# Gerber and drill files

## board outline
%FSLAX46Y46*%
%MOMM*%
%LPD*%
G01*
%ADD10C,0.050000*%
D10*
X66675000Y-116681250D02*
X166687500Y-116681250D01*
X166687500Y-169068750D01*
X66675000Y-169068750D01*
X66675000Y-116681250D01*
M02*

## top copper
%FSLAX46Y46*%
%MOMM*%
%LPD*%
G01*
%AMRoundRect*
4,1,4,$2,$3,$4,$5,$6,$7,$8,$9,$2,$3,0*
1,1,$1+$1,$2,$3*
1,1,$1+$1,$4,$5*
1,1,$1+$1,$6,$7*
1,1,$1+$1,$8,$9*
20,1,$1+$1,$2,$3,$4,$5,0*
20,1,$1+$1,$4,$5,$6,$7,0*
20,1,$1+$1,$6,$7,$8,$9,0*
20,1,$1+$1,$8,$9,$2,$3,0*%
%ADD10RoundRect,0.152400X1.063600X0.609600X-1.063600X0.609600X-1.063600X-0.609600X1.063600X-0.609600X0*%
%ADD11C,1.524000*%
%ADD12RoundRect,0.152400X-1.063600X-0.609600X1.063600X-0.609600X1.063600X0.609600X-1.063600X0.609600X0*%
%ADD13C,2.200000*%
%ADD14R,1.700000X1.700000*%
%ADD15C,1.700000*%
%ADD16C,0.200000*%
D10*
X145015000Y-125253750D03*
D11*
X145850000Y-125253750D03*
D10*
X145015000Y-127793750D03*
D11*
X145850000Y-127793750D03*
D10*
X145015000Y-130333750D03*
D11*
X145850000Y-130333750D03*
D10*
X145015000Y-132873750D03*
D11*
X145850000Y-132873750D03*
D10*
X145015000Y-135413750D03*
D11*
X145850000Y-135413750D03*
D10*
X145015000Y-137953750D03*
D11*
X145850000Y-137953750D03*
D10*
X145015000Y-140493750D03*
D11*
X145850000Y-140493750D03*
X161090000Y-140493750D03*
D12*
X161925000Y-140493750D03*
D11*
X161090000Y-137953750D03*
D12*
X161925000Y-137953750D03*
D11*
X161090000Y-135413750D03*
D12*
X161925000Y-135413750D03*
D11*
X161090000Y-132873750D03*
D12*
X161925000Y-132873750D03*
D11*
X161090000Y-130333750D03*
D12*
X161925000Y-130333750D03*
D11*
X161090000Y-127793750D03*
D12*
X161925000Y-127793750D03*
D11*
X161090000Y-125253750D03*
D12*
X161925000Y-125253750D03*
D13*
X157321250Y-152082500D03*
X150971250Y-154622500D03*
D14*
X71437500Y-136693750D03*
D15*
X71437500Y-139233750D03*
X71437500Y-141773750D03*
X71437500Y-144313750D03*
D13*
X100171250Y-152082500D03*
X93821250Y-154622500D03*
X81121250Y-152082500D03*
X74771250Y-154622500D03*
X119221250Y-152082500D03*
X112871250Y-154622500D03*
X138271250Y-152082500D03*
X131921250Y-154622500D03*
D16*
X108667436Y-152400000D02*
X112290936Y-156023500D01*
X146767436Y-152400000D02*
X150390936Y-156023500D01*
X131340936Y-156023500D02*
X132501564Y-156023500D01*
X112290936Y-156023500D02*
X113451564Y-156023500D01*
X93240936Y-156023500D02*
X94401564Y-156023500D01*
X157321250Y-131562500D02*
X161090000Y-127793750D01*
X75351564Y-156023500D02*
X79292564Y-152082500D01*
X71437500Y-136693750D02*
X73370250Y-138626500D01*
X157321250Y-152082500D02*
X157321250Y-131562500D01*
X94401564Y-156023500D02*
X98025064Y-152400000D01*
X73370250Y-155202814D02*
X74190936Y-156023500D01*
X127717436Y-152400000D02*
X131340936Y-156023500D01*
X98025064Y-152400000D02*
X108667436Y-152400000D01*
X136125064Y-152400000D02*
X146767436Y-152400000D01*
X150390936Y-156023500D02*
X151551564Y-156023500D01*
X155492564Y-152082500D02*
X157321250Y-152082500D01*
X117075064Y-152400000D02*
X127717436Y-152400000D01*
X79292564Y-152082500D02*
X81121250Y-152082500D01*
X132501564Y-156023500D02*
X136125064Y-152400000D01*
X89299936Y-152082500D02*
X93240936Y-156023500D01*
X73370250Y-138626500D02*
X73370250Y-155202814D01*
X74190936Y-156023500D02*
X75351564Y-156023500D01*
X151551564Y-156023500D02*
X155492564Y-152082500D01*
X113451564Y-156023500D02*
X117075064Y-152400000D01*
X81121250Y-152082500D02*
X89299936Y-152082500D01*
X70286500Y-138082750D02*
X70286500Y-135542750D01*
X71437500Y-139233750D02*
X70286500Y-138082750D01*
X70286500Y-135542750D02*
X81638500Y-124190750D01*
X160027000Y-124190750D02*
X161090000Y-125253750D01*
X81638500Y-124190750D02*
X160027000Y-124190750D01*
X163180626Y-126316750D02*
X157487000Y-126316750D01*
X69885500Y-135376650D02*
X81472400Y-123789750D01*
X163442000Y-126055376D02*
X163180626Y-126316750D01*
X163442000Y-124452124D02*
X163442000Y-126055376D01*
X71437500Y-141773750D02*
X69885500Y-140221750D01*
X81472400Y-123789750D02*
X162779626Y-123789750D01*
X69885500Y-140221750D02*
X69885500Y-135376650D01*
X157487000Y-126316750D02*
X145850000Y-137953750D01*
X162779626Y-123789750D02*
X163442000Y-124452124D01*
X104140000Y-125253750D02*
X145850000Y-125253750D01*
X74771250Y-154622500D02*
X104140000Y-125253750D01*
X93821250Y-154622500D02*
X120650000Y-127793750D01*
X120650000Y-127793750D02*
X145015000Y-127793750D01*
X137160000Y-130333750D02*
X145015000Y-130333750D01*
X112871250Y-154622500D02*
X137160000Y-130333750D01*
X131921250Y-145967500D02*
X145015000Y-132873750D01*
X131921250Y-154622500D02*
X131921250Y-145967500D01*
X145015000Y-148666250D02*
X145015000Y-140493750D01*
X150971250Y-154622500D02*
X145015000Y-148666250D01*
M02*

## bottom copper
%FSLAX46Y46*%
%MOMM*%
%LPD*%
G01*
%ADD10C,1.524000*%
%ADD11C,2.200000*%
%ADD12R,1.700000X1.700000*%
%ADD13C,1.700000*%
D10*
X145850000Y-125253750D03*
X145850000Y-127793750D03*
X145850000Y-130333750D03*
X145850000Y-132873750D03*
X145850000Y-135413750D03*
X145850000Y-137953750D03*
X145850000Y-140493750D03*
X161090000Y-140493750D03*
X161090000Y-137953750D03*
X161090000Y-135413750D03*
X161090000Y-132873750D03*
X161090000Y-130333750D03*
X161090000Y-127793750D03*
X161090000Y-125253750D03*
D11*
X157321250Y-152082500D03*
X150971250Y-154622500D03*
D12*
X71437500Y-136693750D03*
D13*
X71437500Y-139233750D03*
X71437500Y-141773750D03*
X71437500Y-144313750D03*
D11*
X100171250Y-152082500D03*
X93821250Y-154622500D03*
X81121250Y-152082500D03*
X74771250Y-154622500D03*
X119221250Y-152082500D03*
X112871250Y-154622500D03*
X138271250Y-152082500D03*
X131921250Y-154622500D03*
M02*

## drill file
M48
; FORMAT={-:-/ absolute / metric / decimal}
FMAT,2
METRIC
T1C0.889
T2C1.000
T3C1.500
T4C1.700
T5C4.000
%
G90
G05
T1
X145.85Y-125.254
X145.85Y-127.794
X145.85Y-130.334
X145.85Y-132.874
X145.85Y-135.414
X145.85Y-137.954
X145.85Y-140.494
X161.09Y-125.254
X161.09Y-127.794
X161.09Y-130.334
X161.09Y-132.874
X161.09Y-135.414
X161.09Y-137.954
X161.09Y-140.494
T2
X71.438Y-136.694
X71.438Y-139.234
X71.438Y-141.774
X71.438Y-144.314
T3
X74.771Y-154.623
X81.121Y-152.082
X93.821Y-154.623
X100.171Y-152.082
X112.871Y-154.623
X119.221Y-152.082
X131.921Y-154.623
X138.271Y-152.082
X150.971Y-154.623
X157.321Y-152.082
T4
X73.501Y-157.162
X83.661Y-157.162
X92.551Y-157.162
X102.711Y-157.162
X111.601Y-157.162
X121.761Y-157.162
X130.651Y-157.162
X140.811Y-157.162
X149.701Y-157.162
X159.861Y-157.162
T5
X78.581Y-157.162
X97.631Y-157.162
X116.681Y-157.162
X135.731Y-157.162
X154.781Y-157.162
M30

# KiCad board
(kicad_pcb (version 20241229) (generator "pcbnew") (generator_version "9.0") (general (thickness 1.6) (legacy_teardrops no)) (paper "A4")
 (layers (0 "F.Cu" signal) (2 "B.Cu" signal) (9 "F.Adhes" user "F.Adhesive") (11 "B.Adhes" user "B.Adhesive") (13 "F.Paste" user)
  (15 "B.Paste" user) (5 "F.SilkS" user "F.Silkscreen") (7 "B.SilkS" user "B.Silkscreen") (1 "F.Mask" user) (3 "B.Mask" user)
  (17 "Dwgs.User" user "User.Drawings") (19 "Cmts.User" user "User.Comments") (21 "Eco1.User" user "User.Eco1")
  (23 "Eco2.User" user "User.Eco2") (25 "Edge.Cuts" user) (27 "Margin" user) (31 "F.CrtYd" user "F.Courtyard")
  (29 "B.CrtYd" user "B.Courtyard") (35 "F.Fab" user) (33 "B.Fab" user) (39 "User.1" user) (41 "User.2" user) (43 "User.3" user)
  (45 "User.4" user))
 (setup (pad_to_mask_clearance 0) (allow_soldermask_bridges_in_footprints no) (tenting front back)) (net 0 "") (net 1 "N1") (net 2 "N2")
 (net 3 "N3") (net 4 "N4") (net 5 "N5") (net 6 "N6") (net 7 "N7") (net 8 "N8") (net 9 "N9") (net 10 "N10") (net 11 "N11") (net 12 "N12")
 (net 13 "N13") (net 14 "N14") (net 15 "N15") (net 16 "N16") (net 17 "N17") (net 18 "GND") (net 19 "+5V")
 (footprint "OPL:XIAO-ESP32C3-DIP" (layer "F.Cu") (at 153.59 132.87375)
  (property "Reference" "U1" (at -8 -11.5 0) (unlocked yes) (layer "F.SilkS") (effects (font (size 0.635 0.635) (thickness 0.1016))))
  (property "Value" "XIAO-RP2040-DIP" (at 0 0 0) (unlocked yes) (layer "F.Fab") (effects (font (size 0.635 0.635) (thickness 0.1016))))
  (pad "1" smd roundrect (at -8.575 -7.62 180) (size 2.432 1.524) (layers "F.Cu" "F.Mask") (roundrect_rratio 0.1) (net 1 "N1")
   (thermal_bridge_angle 45))
  (pad "1" thru_hole circle (at -7.74 -7.62 180) (size 1.524 1.524) (drill 0.889) (layers "*.Cu" "*.Mask") (remove_unused_layers no)
   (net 1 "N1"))
  (pad "2" smd roundrect (at -8.575 -5.08 180) (size 2.432 1.524) (layers "F.Cu" "F.Mask") (roundrect_rratio 0.1) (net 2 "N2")
   (thermal_bridge_angle 45))
  (pad "2" thru_hole circle (at -7.74 -5.08 180) (size 1.524 1.524) (drill 0.889) (layers "*.Cu" "*.Mask") (remove_unused_layers no)
   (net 2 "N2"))
  (pad "3" smd roundrect (at -8.575 -2.54 180) (size 2.432 1.524) (layers "F.Cu" "F.Mask") (roundrect_rratio 0.1) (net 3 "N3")
   (thermal_bridge_angle 45))
  (pad "3" thru_hole circle (at -7.74 -2.54 180) (size 1.524 1.524) (drill 0.889) (layers "*.Cu" "*.Mask") (remove_unused_layers no)
   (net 3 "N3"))
  (pad "4" smd roundrect (at -8.575 0 180) (size 2.432 1.524) (layers "F.Cu" "F.Mask") (roundrect_rratio 0.1) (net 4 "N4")
   (thermal_bridge_angle 45))
  (pad "4" thru_hole circle (at -7.74 0 180) (size 1.524 1.524) (drill 0.889) (layers "*.Cu" "*.Mask") (remove_unused_layers no)
   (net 4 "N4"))
  (pad "5" smd roundrect (at -8.575 2.54 180) (size 2.432 1.524) (layers "F.Cu" "F.Mask") (roundrect_rratio 0.1) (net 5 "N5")
   (thermal_bridge_angle 45))
  (pad "5" thru_hole circle (at -7.74 2.54 180) (size 1.524 1.524) (drill 0.889) (layers "*.Cu" "*.Mask") (remove_unused_layers no)
   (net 5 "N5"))
  (pad "6" smd roundrect (at -8.575 5.08 180) (size 2.432 1.524) (layers "F.Cu" "F.Mask") (roundrect_rratio 0.1) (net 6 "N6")
   (thermal_bridge_angle 45))
  (pad "6" thru_hole circle (at -7.74 5.08 180) (size 1.524 1.524) (drill 0.889) (layers "*.Cu" "*.Mask") (remove_unused_layers no)
   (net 6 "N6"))
  (pad "7" smd roundrect (at -8.575 7.62 180) (size 2.432 1.524) (layers "F.Cu" "F.Mask") (roundrect_rratio 0.1) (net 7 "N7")
   (thermal_bridge_angle 45))
  (pad "7" thru_hole circle (at -7.74 7.62 180) (size 1.524 1.524) (drill 0.889) (layers "*.Cu" "*.Mask") (remove_unused_layers no)
   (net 7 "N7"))
  (pad "8" thru_hole circle (at 7.5 7.62) (size 1.524 1.524) (drill 0.889) (layers "*.Cu" "*.Mask") (remove_unused_layers no) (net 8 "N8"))
  (pad "8" smd roundrect (at 8.335 7.62) (size 2.432 1.524) (layers "F.Cu" "F.Mask") (roundrect_rratio 0.1) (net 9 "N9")
   (thermal_bridge_angle 45))
  (pad "9" thru_hole circle (at 7.5 5.08) (size 1.524 1.524) (drill 0.889) (layers "*.Cu" "*.Mask") (remove_unused_layers no) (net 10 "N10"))
  (pad "9" smd roundrect (at 8.335 5.08) (size 2.432 1.524) (layers "F.Cu" "F.Mask") (roundrect_rratio 0.1) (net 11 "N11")
   (thermal_bridge_angle 45))
  (pad "10" thru_hole circle (at 7.5 2.54) (size 1.524 1.524) (drill 0.889) (layers "*.Cu" "*.Mask") (remove_unused_layers no)
   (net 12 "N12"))
  (pad "10" smd roundrect (at 8.335 2.54) (size 2.432 1.524) (layers "F.Cu" "F.Mask") (roundrect_rratio 0.1) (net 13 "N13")
   (thermal_bridge_angle 45))
  (pad "11" thru_hole circle (at 7.5 0) (size 1.524 1.524) (drill 0.889) (layers "*.Cu" "*.Mask") (remove_unused_layers no) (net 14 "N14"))
  (pad "11" smd roundrect (at 8.335 0) (size 2.432 1.524) (layers "F.Cu" "F.Mask") (roundrect_rratio 0.1) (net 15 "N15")
   (thermal_bridge_angle 45))
  (pad "12" thru_hole circle (at 7.5 -2.54) (size 1.524 1.524) (drill 0.889) (layers "*.Cu" "*.Mask") (remove_unused_layers no)
   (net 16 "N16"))
  (pad "12" smd roundrect (at 8.335 -2.54) (size 2.432 1.524) (layers "F.Cu" "F.Mask") (roundrect_rratio 0.1) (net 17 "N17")
   (thermal_bridge_angle 45))
  (pad "13" thru_hole circle (at 7.5 -5.08) (size 1.524 1.524) (drill 0.889) (layers "*.Cu" "*.Mask") (remove_unused_layers no)
   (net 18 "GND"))
  (pad "13" smd roundrect (at 8.335 -5.08) (size 2.432 1.524) (layers "F.Cu" "F.Mask") (roundrect_rratio 0.1) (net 18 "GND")
   (thermal_bridge_angle 45))
  (pad "14" thru_hole circle (at 7.5 -7.62) (size 1.524 1.524) (drill 0.889) (layers "*.Cu" "*.Mask") (remove_unused_layers no)
   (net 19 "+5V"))
  (pad "14" smd roundrect (at 8.335 -7.62) (size 2.432 1.524) (layers "F.Cu" "F.Mask") (roundrect_rratio 0.1) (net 19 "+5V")
   (thermal_bridge_angle 45)))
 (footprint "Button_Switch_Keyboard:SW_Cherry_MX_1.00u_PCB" (layer "F.Cu") (at 157.32125 152.0825)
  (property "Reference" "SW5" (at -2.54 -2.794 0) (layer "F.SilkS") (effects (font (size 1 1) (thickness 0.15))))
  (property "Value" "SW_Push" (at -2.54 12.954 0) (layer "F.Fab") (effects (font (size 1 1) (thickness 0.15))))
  (pad "" np_thru_hole circle (at -7.62 5.08) (size 1.7 1.7) (drill 1.7) (layers "*.Cu" "*.Mask"))
  (pad "" np_thru_hole circle (at -2.54 5.08) (size 4 4) (drill 4) (layers "*.Cu" "*.Mask"))
  (pad "" np_thru_hole circle (at 2.54 5.08) (size 1.7 1.7) (drill 1.7) (layers "*.Cu" "*.Mask"))
  (pad "1" thru_hole circle (at 0 0) (size 2.2 2.2) (drill 1.5) (layers "*.Cu" "*.Mask") (remove_unused_layers no) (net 18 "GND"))
  (pad "2" thru_hole circle (at -6.35 2.54) (size 2.2 2.2) (drill 1.5) (layers "*.Cu" "*.Mask") (remove_unused_layers no) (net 7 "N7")))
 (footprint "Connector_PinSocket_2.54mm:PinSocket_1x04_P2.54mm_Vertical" (layer "F.Cu") (at 71.4375 136.69375)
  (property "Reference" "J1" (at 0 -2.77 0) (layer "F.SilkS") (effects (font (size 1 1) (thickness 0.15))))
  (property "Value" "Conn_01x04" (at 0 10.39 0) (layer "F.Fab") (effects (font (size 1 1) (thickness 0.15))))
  (pad "1" thru_hole rect (at 0 0) (size 1.7 1.7) (drill 1) (layers "*.Cu" "*.Mask") (remove_unused_layers no) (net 18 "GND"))
  (pad "2" thru_hole circle (at 0 2.54) (size 1.7 1.7) (drill 1) (layers "*.Cu" "*.Mask") (remove_unused_layers no) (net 19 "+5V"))
  (pad "3" thru_hole circle (at 0 5.08) (size 1.7 1.7) (drill 1) (layers "*.Cu" "*.Mask") (remove_unused_layers no) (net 6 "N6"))
  (pad "4" thru_hole circle (at 0 7.62) (size 1.7 1.7) (drill 1) (layers "*.Cu" "*.Mask") (remove_unused_layers no) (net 5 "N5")))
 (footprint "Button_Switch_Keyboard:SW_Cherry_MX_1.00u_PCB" (layer "F.Cu") (at 100.17125 152.0825)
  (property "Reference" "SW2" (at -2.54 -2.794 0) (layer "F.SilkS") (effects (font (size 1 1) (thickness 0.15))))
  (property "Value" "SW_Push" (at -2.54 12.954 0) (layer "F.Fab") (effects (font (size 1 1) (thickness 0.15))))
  (pad "" np_thru_hole circle (at -7.62 5.08) (size 1.7 1.7) (drill 1.7) (layers "*.Cu" "*.Mask"))
  (pad "" np_thru_hole circle (at -2.54 5.08) (size 4 4) (drill 4) (layers "*.Cu" "*.Mask"))
  (pad "" np_thru_hole circle (at 2.54 5.08) (size 1.7 1.7) (drill 1.7) (layers "*.Cu" "*.Mask"))
  (pad "1" thru_hole circle (at 0 0) (size 2.2 2.2) (drill 1.5) (layers "*.Cu" "*.Mask") (remove_unused_layers no) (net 18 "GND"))
  (pad "2" thru_hole circle (at -6.35 2.54) (size 2.2 2.2) (drill 1.5) (layers "*.Cu" "*.Mask") (remove_unused_layers no) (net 2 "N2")))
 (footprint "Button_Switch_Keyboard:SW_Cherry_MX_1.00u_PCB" (layer "F.Cu") (at 81.12125 152.0825)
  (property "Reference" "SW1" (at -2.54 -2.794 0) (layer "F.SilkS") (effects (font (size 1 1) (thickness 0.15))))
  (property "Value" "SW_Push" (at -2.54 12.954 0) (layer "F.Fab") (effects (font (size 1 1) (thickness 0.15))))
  (pad "" np_thru_hole circle (at -7.62 5.08) (size 1.7 1.7) (drill 1.7) (layers "*.Cu" "*.Mask"))
  (pad "" np_thru_hole circle (at -2.54 5.08) (size 4 4) (drill 4) (layers "*.Cu" "*.Mask"))
  (pad "" np_thru_hole circle (at 2.54 5.08) (size 1.7 1.7) (drill 1.7) (layers "*.Cu" "*.Mask"))
  (pad "1" thru_hole circle (at 0 0) (size 2.2 2.2) (drill 1.5) (layers "*.Cu" "*.Mask") (remove_unused_layers no) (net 18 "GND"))
  (pad "2" thru_hole circle (at -6.35 2.54) (size 2.2 2.2) (drill 1.5) (layers "*.Cu" "*.Mask") (remove_unused_layers no) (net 1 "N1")))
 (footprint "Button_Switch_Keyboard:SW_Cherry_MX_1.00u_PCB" (layer "F.Cu") (at 119.22125 152.0825)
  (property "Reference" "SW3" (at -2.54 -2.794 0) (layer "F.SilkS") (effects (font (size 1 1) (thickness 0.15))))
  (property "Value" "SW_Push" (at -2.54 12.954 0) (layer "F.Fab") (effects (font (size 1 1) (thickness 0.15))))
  (pad "" np_thru_hole circle (at -7.62 5.08) (size 1.7 1.7) (drill 1.7) (layers "*.Cu" "*.Mask"))
  (pad "" np_thru_hole circle (at -2.54 5.08) (size 4 4) (drill 4) (layers "*.Cu" "*.Mask"))
  (pad "" np_thru_hole circle (at 2.54 5.08) (size 1.7 1.7) (drill 1.7) (layers "*.Cu" "*.Mask"))
  (pad "1" thru_hole circle (at 0 0) (size 2.2 2.2) (drill 1.5) (layers "*.Cu" "*.Mask") (remove_unused_layers no) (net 18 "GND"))
  (pad "2" thru_hole circle (at -6.35 2.54) (size 2.2 2.2) (drill 1.5) (layers "*.Cu" "*.Mask") (remove_unused_layers no) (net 3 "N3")))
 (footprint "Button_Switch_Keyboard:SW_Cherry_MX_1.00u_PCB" (layer "F.Cu") (at 138.27125 152.0825)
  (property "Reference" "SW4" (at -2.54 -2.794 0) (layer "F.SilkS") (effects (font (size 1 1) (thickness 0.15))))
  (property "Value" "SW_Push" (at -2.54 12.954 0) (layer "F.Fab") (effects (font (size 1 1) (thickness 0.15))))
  (pad "" np_thru_hole circle (at -7.62 5.08) (size 1.7 1.7) (drill 1.7) (layers "*.Cu" "*.Mask"))
  (pad "" np_thru_hole circle (at -2.54 5.08) (size 4 4) (drill 4) (layers "*.Cu" "*.Mask"))
  (pad "" np_thru_hole circle (at 2.54 5.08) (size 1.7 1.7) (drill 1.7) (layers "*.Cu" "*.Mask"))
  (pad "1" thru_hole circle (at 0 0) (size 2.2 2.2) (drill 1.5) (layers "*.Cu" "*.Mask") (remove_unused_layers no) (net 18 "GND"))
  (pad "2" thru_hole circle (at -6.35 2.54) (size 2.2 2.2) (drill 1.5) (layers "*.Cu" "*.Mask") (remove_unused_layers no) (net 4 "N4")))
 (gr_rect (start 66.675 116.68125) (end 166.6875 169.06875) (stroke (width 0.05) (type default)) (fill no) (layer "Edge.Cuts"))
 (segment (start 108.667436 152.4) (end 112.290936 156.0235) (width 0.2) (layer "F.Cu") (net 18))
 (segment (start 146.767436 152.4) (end 150.390936 156.0235) (width 0.2) (layer "F.Cu") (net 18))
 (segment (start 131.340936 156.0235) (end 132.501564 156.0235) (width 0.2) (layer "F.Cu") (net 18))
 (segment (start 112.290936 156.0235) (end 113.451564 156.0235) (width 0.2) (layer "F.Cu") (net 18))
 (segment (start 93.240936 156.0235) (end 94.401564 156.0235) (width 0.2) (layer "F.Cu") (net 18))
 (segment (start 157.32125 131.5625) (end 161.09 127.79375) (width 0.2) (layer "F.Cu") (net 18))
 (segment (start 75.351564 156.0235) (end 79.292564 152.0825) (width 0.2) (layer "F.Cu") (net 18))
 (segment (start 71.4375 136.69375) (end 73.37025 138.6265) (width 0.2) (layer "F.Cu") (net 18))
 (segment (start 157.32125 152.0825) (end 157.32125 131.5625) (width 0.2) (layer "F.Cu") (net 18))
 (segment (start 94.401564 156.0235) (end 98.025064 152.4) (width 0.2) (layer "F.Cu") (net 18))
 (segment (start 73.37025 155.202814) (end 74.190936 156.0235) (width 0.2) (layer "F.Cu") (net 18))
 (segment (start 127.717436 152.4) (end 131.340936 156.0235) (width 0.2) (layer "F.Cu") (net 18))
 (segment (start 98.025064 152.4) (end 108.667436 152.4) (width 0.2) (layer "F.Cu") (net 18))
 (segment (start 136.125064 152.4) (end 146.767436 152.4) (width 0.2) (layer "F.Cu") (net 18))
 (segment (start 150.390936 156.0235) (end 151.551564 156.0235) (width 0.2) (layer "F.Cu") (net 18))
 (segment (start 155.492564 152.0825) (end 157.32125 152.0825) (width 0.2) (layer "F.Cu") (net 18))
 (segment (start 117.075064 152.4) (end 127.717436 152.4) (width 0.2) (layer "F.Cu") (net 18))
 (segment (start 79.292564 152.0825) (end 81.12125 152.0825) (width 0.2) (layer "F.Cu") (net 18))
 (segment (start 132.501564 156.0235) (end 136.125064 152.4) (width 0.2) (layer "F.Cu") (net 18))
 (segment (start 89.299936 152.0825) (end 93.240936 156.0235) (width 0.2) (layer "F.Cu") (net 18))
 (segment (start 73.37025 138.6265) (end 73.37025 155.202814) (width 0.2) (layer "F.Cu") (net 18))
 (segment (start 74.190936 156.0235) (end 75.351564 156.0235) (width 0.2) (layer "F.Cu") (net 18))
 (segment (start 151.551564 156.0235) (end 155.492564 152.0825) (width 0.2) (layer "F.Cu") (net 18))
 (segment (start 113.451564 156.0235) (end 117.075064 152.4) (width 0.2) (layer "F.Cu") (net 18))
 (segment (start 81.12125 152.0825) (end 89.299936 152.0825) (width 0.2) (layer "F.Cu") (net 18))
 (segment (start 70.2865 138.08275) (end 70.2865 135.54275) (width 0.2) (layer "F.Cu") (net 19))
 (segment (start 71.4375 139.23375) (end 70.2865 138.08275) (width 0.2) (layer "F.Cu") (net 19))
 (segment (start 70.2865 135.54275) (end 81.6385 124.19075) (width 0.2) (layer "F.Cu") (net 19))
 (segment (start 160.027 124.19075) (end 161.09 125.25375) (width 0.2) (layer "F.Cu") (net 19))
 (segment (start 81.6385 124.19075) (end 160.027 124.19075) (width 0.2) (layer "F.Cu") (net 19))
 (segment (start 163.180626 126.31675) (end 157.487 126.31675) (width 0.2) (layer "F.Cu") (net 6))
 (segment (start 69.8855 135.37665) (end 81.4724 123.78975) (width 0.2) (layer "F.Cu") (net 6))
 (segment (start 163.442 126.055376) (end 163.180626 126.31675) (width 0.2) (layer "F.Cu") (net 6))
 (segment (start 163.442 124.452124) (end 163.442 126.055376) (width 0.2) (layer "F.Cu") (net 6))
 (segment (start 71.4375 141.77375) (end 69.8855 140.22175) (width 0.2) (layer "F.Cu") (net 6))
 (segment (start 81.4724 123.78975) (end 162.779626 123.78975) (width 0.2) (layer "F.Cu") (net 6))
 (segment (start 69.8855 140.22175) (end 69.8855 135.37665) (width 0.2) (layer "F.Cu") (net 6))
 (segment (start 157.487 126.31675) (end 145.85 137.95375) (width 0.2) (layer "F.Cu") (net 6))
 (segment (start 162.779626 123.78975) (end 163.442 124.452124) (width 0.2) (layer "F.Cu") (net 6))
 (segment (start 104.14 125.25375) (end 145.85 125.25375) (width 0.2) (layer "F.Cu") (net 1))
 (segment (start 74.77125 154.6225) (end 104.14 125.25375) (width 0.2) (layer "F.Cu") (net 1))
 (segment (start 93.82125 154.6225) (end 120.65 127.79375) (width 0.2) (layer "F.Cu") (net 2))
 (segment (start 120.65 127.79375) (end 145.015 127.79375) (width 0.2) (layer "F.Cu") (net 2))
 (segment (start 137.16 130.33375) (end 145.015 130.33375) (width 0.2) (layer "F.Cu") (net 3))
 (segment (start 112.87125 154.6225) (end 137.16 130.33375) (width 0.2) (layer "F.Cu") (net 3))
 (segment (start 131.92125 145.9675) (end 145.015 132.87375) (width 0.2) (layer "F.Cu") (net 4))
 (segment (start 131.92125 154.6225) (end 131.92125 145.9675) (width 0.2) (layer "F.Cu") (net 4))
 (segment (start 145.015 148.66625) (end 145.015 140.49375) (width 0.2) (layer "F.Cu") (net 7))
 (segment (start 150.97125 154.6225) (end 145.015 148.66625) (width 0.2) (layer "F.Cu") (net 7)))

